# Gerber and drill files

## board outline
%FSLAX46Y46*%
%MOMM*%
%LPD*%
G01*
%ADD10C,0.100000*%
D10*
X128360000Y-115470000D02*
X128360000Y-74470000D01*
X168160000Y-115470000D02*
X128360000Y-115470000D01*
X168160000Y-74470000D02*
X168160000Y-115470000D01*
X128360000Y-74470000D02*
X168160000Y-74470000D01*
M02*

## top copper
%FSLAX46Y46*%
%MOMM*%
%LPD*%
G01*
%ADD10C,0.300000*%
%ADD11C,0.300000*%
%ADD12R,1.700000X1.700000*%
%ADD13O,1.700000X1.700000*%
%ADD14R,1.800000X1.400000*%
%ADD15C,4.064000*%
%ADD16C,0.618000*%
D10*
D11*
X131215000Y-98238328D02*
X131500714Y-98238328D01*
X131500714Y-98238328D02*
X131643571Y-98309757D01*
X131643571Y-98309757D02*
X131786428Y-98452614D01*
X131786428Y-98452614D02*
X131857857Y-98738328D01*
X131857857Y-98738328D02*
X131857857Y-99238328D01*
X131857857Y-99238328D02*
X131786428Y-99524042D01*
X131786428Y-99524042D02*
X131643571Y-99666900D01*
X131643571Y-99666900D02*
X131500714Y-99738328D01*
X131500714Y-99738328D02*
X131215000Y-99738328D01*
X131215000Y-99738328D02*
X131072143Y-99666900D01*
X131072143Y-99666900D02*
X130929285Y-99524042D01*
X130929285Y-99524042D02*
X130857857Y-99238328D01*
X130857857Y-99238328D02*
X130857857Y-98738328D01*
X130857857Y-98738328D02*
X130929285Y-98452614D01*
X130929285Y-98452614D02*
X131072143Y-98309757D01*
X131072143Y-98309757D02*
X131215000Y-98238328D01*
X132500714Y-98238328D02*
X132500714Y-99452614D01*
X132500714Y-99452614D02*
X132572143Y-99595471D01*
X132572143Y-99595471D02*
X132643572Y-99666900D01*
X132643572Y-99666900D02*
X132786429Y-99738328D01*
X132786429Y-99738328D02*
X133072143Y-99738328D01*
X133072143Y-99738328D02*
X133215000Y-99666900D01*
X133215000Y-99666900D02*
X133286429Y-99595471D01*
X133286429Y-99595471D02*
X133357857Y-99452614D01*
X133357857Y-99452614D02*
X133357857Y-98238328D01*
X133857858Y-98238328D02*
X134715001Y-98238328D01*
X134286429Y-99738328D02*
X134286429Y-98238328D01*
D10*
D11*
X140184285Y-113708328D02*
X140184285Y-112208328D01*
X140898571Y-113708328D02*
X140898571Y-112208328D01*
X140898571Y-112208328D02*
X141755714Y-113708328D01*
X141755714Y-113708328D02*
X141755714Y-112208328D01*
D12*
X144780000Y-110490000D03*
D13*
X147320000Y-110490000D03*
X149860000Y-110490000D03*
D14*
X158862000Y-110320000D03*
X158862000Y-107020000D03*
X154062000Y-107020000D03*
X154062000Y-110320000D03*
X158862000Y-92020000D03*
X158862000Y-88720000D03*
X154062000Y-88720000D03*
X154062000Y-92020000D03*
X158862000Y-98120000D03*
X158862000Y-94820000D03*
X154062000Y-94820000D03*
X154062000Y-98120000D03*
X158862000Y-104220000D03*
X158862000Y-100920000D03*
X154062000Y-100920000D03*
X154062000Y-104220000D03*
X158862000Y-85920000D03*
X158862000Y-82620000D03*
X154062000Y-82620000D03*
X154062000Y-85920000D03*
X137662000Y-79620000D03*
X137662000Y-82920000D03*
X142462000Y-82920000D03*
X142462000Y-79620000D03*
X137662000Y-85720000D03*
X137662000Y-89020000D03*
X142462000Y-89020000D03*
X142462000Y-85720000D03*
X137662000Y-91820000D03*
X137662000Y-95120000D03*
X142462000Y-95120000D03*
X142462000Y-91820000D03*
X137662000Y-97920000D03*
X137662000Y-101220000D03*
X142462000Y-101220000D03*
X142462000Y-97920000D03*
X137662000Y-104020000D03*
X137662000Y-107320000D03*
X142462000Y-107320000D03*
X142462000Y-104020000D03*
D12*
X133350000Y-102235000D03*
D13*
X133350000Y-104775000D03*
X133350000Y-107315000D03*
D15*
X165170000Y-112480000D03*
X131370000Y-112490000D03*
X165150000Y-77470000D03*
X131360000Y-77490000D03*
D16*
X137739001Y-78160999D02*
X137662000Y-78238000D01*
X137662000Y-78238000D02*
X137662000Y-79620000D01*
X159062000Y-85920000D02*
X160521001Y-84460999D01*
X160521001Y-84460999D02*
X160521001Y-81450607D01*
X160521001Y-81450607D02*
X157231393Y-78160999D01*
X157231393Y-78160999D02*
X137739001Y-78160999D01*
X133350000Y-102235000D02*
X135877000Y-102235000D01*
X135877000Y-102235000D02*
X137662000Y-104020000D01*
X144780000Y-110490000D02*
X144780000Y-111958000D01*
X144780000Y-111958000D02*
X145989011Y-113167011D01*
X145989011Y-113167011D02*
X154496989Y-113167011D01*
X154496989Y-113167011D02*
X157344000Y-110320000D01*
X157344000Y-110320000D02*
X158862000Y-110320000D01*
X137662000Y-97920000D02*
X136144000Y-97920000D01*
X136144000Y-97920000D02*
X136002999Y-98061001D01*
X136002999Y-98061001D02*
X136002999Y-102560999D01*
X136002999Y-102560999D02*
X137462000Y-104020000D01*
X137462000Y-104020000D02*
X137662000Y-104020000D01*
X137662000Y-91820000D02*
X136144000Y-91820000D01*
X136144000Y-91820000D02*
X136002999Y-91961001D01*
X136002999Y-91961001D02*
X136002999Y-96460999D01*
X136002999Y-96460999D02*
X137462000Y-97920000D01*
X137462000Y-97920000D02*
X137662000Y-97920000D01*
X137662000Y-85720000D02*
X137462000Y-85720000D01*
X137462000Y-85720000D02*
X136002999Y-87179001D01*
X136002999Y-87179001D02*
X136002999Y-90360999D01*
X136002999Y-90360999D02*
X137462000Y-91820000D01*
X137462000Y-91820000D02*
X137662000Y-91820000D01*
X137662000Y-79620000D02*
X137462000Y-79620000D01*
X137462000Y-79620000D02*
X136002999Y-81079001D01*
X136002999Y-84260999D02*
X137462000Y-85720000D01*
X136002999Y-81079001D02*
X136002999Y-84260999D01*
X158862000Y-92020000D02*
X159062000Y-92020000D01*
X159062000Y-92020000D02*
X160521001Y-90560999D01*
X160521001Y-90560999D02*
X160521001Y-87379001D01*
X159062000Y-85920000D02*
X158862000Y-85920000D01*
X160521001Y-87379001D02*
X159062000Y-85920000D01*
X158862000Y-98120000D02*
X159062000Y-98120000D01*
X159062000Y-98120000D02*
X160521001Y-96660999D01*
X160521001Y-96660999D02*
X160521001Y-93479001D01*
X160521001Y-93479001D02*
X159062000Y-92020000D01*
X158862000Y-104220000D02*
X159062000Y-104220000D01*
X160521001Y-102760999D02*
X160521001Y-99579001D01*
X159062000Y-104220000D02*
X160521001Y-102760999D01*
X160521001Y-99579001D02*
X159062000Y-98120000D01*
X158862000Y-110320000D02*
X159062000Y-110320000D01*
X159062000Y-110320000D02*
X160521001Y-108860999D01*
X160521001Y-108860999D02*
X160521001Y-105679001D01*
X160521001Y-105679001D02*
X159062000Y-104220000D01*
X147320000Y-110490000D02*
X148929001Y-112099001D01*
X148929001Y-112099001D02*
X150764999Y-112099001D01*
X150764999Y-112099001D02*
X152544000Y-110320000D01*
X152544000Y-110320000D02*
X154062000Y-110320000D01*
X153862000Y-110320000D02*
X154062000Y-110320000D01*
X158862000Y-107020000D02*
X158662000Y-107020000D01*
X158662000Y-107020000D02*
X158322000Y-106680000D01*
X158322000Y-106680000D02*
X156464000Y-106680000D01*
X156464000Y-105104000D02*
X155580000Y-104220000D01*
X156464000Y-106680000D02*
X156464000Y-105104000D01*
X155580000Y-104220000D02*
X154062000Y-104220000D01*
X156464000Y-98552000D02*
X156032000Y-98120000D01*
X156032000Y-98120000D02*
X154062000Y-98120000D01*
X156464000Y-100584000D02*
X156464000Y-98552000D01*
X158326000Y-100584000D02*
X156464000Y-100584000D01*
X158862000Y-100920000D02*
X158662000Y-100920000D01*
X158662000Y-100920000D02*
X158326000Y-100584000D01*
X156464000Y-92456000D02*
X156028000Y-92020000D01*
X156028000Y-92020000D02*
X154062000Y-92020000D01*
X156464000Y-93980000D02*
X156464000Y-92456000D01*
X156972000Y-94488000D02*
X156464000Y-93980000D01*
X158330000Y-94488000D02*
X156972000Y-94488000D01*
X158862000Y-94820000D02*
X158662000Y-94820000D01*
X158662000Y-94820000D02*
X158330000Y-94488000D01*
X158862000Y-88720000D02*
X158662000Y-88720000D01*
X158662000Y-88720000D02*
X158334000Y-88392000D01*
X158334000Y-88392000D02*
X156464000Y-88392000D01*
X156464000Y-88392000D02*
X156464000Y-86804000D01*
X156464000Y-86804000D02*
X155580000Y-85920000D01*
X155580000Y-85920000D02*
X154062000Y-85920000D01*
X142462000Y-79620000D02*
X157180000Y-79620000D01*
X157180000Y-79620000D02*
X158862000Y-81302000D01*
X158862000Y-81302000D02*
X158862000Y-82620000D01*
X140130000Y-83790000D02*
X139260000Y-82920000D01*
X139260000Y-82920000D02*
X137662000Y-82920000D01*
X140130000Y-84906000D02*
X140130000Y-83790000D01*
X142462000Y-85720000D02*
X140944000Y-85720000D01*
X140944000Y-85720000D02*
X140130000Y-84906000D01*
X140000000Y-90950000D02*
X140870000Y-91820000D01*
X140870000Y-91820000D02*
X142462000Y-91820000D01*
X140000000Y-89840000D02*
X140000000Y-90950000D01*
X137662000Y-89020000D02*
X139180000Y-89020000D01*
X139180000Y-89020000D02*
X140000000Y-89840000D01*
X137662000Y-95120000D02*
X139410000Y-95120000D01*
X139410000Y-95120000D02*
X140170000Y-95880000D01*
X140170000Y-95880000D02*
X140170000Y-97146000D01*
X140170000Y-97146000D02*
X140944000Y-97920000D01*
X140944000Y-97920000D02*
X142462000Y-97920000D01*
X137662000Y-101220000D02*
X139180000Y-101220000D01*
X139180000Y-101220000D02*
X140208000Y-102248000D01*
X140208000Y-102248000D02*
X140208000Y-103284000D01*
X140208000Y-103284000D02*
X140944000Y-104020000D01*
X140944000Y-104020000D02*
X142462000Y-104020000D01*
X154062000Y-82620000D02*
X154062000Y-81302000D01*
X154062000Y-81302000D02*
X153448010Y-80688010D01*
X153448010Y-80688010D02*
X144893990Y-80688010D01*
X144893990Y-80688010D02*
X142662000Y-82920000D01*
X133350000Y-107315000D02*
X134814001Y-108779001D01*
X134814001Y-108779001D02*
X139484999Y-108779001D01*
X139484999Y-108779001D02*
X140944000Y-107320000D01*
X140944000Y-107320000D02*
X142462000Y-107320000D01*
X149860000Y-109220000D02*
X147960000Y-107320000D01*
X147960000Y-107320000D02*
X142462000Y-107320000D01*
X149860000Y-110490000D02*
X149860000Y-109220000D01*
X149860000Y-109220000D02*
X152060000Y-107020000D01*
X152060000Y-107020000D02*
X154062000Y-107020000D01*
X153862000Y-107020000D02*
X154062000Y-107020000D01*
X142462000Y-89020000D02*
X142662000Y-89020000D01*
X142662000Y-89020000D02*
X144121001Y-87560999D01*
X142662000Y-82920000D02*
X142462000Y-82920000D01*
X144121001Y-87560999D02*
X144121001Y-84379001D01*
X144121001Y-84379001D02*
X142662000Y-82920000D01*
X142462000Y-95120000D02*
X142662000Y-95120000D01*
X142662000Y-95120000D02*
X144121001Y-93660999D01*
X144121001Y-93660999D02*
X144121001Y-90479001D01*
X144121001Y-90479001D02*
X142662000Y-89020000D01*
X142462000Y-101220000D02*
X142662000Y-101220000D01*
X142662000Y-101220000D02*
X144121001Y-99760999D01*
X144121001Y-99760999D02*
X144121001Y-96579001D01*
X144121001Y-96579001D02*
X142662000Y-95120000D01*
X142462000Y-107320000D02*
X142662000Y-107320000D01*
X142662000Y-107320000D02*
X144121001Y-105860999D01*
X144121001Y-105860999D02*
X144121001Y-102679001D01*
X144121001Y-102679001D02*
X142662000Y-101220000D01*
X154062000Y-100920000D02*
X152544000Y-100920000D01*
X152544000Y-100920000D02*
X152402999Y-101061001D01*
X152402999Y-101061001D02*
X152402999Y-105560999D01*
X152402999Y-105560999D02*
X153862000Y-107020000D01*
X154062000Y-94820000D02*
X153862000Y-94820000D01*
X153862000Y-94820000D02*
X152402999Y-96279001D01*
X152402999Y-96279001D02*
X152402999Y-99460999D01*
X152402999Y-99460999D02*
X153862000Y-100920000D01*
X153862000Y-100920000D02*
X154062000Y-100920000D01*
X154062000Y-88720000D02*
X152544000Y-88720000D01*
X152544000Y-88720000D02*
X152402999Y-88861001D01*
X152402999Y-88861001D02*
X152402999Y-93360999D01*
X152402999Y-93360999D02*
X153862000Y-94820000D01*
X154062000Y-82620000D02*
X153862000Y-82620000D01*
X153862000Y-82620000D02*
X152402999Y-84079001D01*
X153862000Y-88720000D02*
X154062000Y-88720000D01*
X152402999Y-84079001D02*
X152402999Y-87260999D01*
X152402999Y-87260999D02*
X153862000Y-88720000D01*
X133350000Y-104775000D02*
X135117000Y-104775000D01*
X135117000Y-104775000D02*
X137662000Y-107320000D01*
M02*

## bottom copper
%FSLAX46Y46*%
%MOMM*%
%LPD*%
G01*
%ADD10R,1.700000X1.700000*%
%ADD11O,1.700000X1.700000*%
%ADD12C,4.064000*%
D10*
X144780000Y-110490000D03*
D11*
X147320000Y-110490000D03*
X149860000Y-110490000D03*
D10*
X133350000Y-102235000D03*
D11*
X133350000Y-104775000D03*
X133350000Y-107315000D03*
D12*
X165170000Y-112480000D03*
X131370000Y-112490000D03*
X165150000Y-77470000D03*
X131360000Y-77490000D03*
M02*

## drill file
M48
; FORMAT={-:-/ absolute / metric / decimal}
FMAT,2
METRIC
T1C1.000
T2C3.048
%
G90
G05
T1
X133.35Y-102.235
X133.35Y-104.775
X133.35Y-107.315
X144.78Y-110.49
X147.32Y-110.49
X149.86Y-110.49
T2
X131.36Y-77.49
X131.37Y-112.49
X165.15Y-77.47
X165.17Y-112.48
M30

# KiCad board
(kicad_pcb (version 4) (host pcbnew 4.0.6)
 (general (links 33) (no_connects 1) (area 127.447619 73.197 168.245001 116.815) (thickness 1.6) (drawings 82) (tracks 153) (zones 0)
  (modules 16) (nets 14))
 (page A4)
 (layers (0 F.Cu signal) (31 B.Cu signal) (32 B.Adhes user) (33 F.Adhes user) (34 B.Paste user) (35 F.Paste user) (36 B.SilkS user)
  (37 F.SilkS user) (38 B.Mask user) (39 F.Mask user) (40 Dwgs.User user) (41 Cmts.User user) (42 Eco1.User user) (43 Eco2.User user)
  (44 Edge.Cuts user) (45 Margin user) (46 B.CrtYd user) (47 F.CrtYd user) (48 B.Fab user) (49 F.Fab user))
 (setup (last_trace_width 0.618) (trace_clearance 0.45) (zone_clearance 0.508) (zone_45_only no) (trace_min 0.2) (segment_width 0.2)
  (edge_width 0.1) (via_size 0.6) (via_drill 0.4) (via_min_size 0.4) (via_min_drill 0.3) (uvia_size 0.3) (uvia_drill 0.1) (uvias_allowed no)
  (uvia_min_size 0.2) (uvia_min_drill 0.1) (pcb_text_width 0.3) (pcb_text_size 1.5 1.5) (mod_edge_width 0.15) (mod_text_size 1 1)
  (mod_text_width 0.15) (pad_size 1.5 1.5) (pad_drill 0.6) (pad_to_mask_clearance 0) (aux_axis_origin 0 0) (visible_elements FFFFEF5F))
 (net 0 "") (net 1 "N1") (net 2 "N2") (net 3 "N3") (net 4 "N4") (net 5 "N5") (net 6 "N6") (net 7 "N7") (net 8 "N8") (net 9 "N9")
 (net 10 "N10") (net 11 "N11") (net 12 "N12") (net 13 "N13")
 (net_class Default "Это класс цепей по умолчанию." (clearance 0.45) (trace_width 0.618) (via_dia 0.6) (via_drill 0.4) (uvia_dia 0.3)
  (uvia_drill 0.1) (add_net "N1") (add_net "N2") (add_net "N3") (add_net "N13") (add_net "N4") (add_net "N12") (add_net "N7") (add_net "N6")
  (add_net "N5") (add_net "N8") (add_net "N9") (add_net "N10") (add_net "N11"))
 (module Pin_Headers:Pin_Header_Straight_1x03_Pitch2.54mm (layer F.Cu) (at 144.78 110.49 90)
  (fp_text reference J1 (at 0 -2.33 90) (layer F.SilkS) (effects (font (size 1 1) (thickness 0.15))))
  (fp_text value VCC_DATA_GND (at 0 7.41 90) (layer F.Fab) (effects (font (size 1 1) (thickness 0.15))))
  (pad 1 thru_hole rect (at 0 0 90) (size 1.7 1.7) (drill 1) (layers *.Cu *.Mask) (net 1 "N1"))
  (pad 2 thru_hole oval (at 0 2.54 90) (size 1.7 1.7) (drill 1) (layers *.Cu *.Mask) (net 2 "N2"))
  (pad 3 thru_hole oval (at 0 5.08 90) (size 1.7 1.7) (drill 1) (layers *.Cu *.Mask) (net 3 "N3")))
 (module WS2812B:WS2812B (layer F.Cu) (at 156.462 108.67 270)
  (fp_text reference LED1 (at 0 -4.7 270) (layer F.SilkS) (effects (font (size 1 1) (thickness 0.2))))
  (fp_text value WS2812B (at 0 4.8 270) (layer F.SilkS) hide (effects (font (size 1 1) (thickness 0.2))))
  (pad 1 smd rect (at 1.65 -2.4 270) (size 1.4 1.8) (layers F.Cu F.Paste F.Mask) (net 1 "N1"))
  (pad 2 smd rect (at -1.65 -2.4 270) (size 1.4 1.8) (layers F.Cu F.Paste F.Mask) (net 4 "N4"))
  (pad 3 smd rect (at -1.65 2.4 270) (size 1.4 1.8) (layers F.Cu F.Paste F.Mask) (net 3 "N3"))
  (pad 4 smd rect (at 1.65 2.4 270) (size 1.4 1.8) (layers F.Cu F.Paste F.Mask) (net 2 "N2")))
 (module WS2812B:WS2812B (layer F.Cu) (at 156.462 90.37 270)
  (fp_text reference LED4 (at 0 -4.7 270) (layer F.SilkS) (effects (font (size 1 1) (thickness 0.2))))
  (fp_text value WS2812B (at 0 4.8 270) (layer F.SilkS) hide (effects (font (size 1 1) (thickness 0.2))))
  (pad 1 smd rect (at 1.65 -2.4 270) (size 1.4 1.8) (layers F.Cu F.Paste F.Mask) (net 1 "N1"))
  (pad 2 smd rect (at -1.65 -2.4 270) (size 1.4 1.8) (layers F.Cu F.Paste F.Mask) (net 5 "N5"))
  (pad 3 smd rect (at -1.65 2.4 270) (size 1.4 1.8) (layers F.Cu F.Paste F.Mask) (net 3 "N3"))
  (pad 4 smd rect (at 1.65 2.4 270) (size 1.4 1.8) (layers F.Cu F.Paste F.Mask) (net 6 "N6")))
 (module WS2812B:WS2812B (layer F.Cu) (at 156.462 96.47 270)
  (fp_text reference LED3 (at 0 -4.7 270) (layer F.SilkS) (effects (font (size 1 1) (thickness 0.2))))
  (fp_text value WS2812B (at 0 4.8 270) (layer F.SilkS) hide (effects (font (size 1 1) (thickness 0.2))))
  (pad 1 smd rect (at 1.65 -2.4 270) (size 1.4 1.8) (layers F.Cu F.Paste F.Mask) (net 1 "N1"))
  (pad 2 smd rect (at -1.65 -2.4 270) (size 1.4 1.8) (layers F.Cu F.Paste F.Mask) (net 6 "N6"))
  (pad 3 smd rect (at -1.65 2.4 270) (size 1.4 1.8) (layers F.Cu F.Paste F.Mask) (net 3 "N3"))
  (pad 4 smd rect (at 1.65 2.4 270) (size 1.4 1.8) (layers F.Cu F.Paste F.Mask) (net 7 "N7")))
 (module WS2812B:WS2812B (layer F.Cu) (at 156.462 102.57 270)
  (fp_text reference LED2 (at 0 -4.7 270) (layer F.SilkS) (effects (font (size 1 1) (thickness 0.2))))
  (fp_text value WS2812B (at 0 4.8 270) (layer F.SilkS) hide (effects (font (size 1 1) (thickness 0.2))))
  (pad 1 smd rect (at 1.65 -2.4 270) (size 1.4 1.8) (layers F.Cu F.Paste F.Mask) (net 1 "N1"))
  (pad 2 smd rect (at -1.65 -2.4 270) (size 1.4 1.8) (layers F.Cu F.Paste F.Mask) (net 7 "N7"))
  (pad 3 smd rect (at -1.65 2.4 270) (size 1.4 1.8) (layers F.Cu F.Paste F.Mask) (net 3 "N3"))
  (pad 4 smd rect (at 1.65 2.4 270) (size 1.4 1.8) (layers F.Cu F.Paste F.Mask) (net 4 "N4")))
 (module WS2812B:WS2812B (layer F.Cu) (at 156.462 84.27 270)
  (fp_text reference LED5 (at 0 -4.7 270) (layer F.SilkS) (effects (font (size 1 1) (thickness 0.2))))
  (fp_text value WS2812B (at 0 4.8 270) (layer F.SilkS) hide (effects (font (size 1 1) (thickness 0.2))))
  (pad 1 smd rect (at 1.65 -2.4 270) (size 1.4 1.8) (layers F.Cu F.Paste F.Mask) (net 1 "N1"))
  (pad 2 smd rect (at -1.65 -2.4 270) (size 1.4 1.8) (layers F.Cu F.Paste F.Mask) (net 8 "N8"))
  (pad 3 smd rect (at -1.65 2.4 270) (size 1.4 1.8) (layers F.Cu F.Paste F.Mask) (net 3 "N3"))
  (pad 4 smd rect (at 1.65 2.4 270) (size 1.4 1.8) (layers F.Cu F.Paste F.Mask) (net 5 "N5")))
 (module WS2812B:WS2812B (layer F.Cu) (at 140.062 81.27 90)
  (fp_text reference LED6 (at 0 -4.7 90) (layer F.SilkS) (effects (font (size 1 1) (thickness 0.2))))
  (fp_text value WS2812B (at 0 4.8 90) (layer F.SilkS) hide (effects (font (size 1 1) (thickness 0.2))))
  (pad 1 smd rect (at 1.65 -2.4 90) (size 1.4 1.8) (layers F.Cu F.Paste F.Mask) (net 1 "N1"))
  (pad 2 smd rect (at -1.65 -2.4 90) (size 1.4 1.8) (layers F.Cu F.Paste F.Mask) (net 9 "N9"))
  (pad 3 smd rect (at -1.65 2.4 90) (size 1.4 1.8) (layers F.Cu F.Paste F.Mask) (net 3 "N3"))
  (pad 4 smd rect (at 1.65 2.4 90) (size 1.4 1.8) (layers F.Cu F.Paste F.Mask) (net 8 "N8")))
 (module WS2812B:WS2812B (layer F.Cu) (at 140.062 87.37 90)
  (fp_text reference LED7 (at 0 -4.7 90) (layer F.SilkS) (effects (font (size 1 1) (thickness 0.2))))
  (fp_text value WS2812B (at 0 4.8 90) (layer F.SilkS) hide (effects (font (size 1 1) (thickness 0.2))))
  (pad 1 smd rect (at 1.65 -2.4 90) (size 1.4 1.8) (layers F.Cu F.Paste F.Mask) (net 1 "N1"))
  (pad 2 smd rect (at -1.65 -2.4 90) (size 1.4 1.8) (layers F.Cu F.Paste F.Mask) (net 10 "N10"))
  (pad 3 smd rect (at -1.65 2.4 90) (size 1.4 1.8) (layers F.Cu F.Paste F.Mask) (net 3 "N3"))
  (pad 4 smd rect (at 1.65 2.4 90) (size 1.4 1.8) (layers F.Cu F.Paste F.Mask) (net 9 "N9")))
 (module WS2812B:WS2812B (layer F.Cu) (at 140.062 93.47 90)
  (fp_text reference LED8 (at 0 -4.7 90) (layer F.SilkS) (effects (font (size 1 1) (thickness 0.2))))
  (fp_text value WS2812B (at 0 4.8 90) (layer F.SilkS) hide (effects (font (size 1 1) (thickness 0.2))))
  (pad 1 smd rect (at 1.65 -2.4 90) (size 1.4 1.8) (layers F.Cu F.Paste F.Mask) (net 1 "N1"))
  (pad 2 smd rect (at -1.65 -2.4 90) (size 1.4 1.8) (layers F.Cu F.Paste F.Mask) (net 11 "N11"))
  (pad 3 smd rect (at -1.65 2.4 90) (size 1.4 1.8) (layers F.Cu F.Paste F.Mask) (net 3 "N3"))
  (pad 4 smd rect (at 1.65 2.4 90) (size 1.4 1.8) (layers F.Cu F.Paste F.Mask) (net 10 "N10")))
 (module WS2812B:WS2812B (layer F.Cu) (at 140.062 99.57 90)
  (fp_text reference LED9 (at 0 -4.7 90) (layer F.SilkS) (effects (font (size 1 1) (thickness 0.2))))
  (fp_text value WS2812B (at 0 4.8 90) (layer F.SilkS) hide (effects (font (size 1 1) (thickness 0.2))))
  (pad 1 smd rect (at 1.65 -2.4 90) (size 1.4 1.8) (layers F.Cu F.Paste F.Mask) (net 1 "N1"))
  (pad 2 smd rect (at -1.65 -2.4 90) (size 1.4 1.8) (layers F.Cu F.Paste F.Mask) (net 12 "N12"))
  (pad 3 smd rect (at -1.65 2.4 90) (size 1.4 1.8) (layers F.Cu F.Paste F.Mask) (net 3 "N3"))
  (pad 4 smd rect (at 1.65 2.4 90) (size 1.4 1.8) (layers F.Cu F.Paste F.Mask) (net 11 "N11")))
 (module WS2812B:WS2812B (layer F.Cu) (at 140.062 105.67 90)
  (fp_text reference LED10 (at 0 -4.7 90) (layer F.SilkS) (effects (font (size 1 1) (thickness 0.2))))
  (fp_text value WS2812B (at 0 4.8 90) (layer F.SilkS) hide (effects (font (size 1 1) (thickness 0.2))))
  (pad 1 smd rect (at 1.65 -2.4 90) (size 1.4 1.8) (layers F.Cu F.Paste F.Mask) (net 1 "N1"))
  (pad 2 smd rect (at -1.65 -2.4 90) (size 1.4 1.8) (layers F.Cu F.Paste F.Mask) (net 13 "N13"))
  (pad 3 smd rect (at -1.65 2.4 90) (size 1.4 1.8) (layers F.Cu F.Paste F.Mask) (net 3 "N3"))
  (pad 4 smd rect (at 1.65 2.4 90) (size 1.4 1.8) (layers F.Cu F.Paste F.Mask) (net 12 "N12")))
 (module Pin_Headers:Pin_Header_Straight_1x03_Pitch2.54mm (layer F.Cu) (at 133.35 102.235)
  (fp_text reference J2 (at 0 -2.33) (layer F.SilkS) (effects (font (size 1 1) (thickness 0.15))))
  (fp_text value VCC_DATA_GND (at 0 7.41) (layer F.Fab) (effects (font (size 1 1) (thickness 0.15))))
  (pad 1 thru_hole rect (at 0 0) (size 1.7 1.7) (drill 1) (layers *.Cu *.Mask) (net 1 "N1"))
  (pad 2 thru_hole oval (at 0 2.54) (size 1.7 1.7) (drill 1) (layers *.Cu *.Mask) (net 13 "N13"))
  (pad 3 thru_hole oval (at 0 5.08) (size 1.7 1.7) (drill 1) (layers *.Cu *.Mask) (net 3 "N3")))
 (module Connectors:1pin (layer F.Cu) (at 165.17 112.48)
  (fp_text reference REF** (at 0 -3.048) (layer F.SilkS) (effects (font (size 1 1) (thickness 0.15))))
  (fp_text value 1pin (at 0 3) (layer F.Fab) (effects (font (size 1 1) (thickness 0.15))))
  (pad 1 thru_hole circle (at 0 0) (size 4.064 4.064) (drill 3.048) (layers *.Cu *.Mask)))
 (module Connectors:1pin (layer F.Cu) (at 131.37 112.49)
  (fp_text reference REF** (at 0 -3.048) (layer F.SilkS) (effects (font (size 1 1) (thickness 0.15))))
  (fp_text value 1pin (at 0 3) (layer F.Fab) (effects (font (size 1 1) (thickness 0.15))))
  (pad 1 thru_hole circle (at 0 0) (size 4.064 4.064) (drill 3.048) (layers *.Cu *.Mask)))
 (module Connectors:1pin (layer F.Cu) (at 165.15 77.47)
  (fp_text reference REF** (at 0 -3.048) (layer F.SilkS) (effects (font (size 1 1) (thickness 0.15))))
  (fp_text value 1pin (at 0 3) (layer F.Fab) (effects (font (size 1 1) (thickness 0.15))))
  (pad 1 thru_hole circle (at 0 0) (size 4.064 4.064) (drill 3.048) (layers *.Cu *.Mask)))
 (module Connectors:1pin (layer F.Cu) (at 131.36 77.49)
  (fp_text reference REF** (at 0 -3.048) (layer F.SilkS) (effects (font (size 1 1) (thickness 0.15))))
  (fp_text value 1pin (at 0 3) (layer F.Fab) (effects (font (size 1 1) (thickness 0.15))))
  (pad 1 thru_hole circle (at 0 0) (size 4.064 4.064) (drill 3.048) (layers *.Cu *.Mask)))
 (gr_line (start 128.36 115.47) (end 128.36 74.47) (layer Edge.Cuts) (width 0.1))
 (gr_line (start 168.16 115.47) (end 128.36 115.47) (layer Edge.Cuts) (width 0.1))
 (gr_line (start 168.16 74.47) (end 168.16 115.47) (layer Edge.Cuts) (width 0.1))
 (gr_line (start 128.36 74.47) (end 168.16 74.47) (layer Edge.Cuts) (width 0.1))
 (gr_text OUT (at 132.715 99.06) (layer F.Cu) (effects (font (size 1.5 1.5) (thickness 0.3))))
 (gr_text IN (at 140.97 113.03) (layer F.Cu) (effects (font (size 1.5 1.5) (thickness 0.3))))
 (segment (start 137.739001 78.160999) (end 137.662 78.238) (width 0.618) (layer F.Cu) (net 1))
 (segment (start 137.662 78.238) (end 137.662 79.62) (width 0.618) (layer F.Cu) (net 1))
 (segment (start 159.062 85.92) (end 160.521001 84.460999) (width 0.618) (layer F.Cu) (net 1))
 (segment (start 160.521001 84.460999) (end 160.521001 81.450607) (width 0.618) (layer F.Cu) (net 1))
 (segment (start 160.521001 81.450607) (end 157.231393 78.160999) (width 0.618) (layer F.Cu) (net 1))
 (segment (start 157.231393 78.160999) (end 137.739001 78.160999) (width 0.618) (layer F.Cu) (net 1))
 (segment (start 133.35 102.235) (end 135.877 102.235) (width 0.618) (layer F.Cu) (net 1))
 (segment (start 135.877 102.235) (end 137.662 104.02) (width 0.618) (layer F.Cu) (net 1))
 (segment (start 144.78 110.49) (end 144.78 111.958) (width 0.618) (layer F.Cu) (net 1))
 (segment (start 144.78 111.958) (end 145.989011 113.167011) (width 0.618) (layer F.Cu) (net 1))
 (segment (start 145.989011 113.167011) (end 154.496989 113.167011) (width 0.618) (layer F.Cu) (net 1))
 (segment (start 154.496989 113.167011) (end 157.344 110.32) (width 0.618) (layer F.Cu) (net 1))
 (segment (start 157.344 110.32) (end 158.862 110.32) (width 0.618) (layer F.Cu) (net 1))
 (segment (start 137.662 97.92) (end 136.144 97.92) (width 0.618) (layer F.Cu) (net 1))
 (segment (start 136.144 97.92) (end 136.002999 98.061001) (width 0.618) (layer F.Cu) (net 1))
 (segment (start 136.002999 98.061001) (end 136.002999 102.560999) (width 0.618) (layer F.Cu) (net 1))
 (segment (start 136.002999 102.560999) (end 137.462 104.02) (width 0.618) (layer F.Cu) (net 1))
 (segment (start 137.462 104.02) (end 137.662 104.02) (width 0.618) (layer F.Cu) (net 1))
 (segment (start 137.662 91.82) (end 136.144 91.82) (width 0.618) (layer F.Cu) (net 1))
 (segment (start 136.144 91.82) (end 136.002999 91.961001) (width 0.618) (layer F.Cu) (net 1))
 (segment (start 136.002999 91.961001) (end 136.002999 96.460999) (width 0.618) (layer F.Cu) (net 1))
 (segment (start 136.002999 96.460999) (end 137.462 97.92) (width 0.618) (layer F.Cu) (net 1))
 (segment (start 137.462 97.92) (end 137.662 97.92) (width 0.618) (layer F.Cu) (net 1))
 (segment (start 137.662 85.72) (end 137.462 85.72) (width 0.618) (layer F.Cu) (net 1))
 (segment (start 137.462 85.72) (end 136.002999 87.179001) (width 0.618) (layer F.Cu) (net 1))
 (segment (start 136.002999 87.179001) (end 136.002999 90.360999) (width 0.618) (layer F.Cu) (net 1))
 (segment (start 136.002999 90.360999) (end 137.462 91.82) (width 0.618) (layer F.Cu) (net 1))
 (segment (start 137.462 91.82) (end 137.662 91.82) (width 0.618) (layer F.Cu) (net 1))
 (segment (start 137.662 79.62) (end 137.462 79.62) (width 0.618) (layer F.Cu) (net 1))
 (segment (start 137.462 79.62) (end 136.002999 81.079001) (width 0.618) (layer F.Cu) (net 1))
 (segment (start 136.002999 84.260999) (end 137.462 85.72) (width 0.618) (layer F.Cu) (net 1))
 (segment (start 136.002999 81.079001) (end 136.002999 84.260999) (width 0.618) (layer F.Cu) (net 1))
 (segment (start 158.862 92.02) (end 159.062 92.02) (width 0.618) (layer F.Cu) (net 1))
 (segment (start 159.062 92.02) (end 160.521001 90.560999) (width 0.618) (layer F.Cu) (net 1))
 (segment (start 160.521001 90.560999) (end 160.521001 87.379001) (width 0.618) (layer F.Cu) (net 1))
 (segment (start 159.062 85.92) (end 158.862 85.92) (width 0.618) (layer F.Cu) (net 1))
 (segment (start 160.521001 87.379001) (end 159.062 85.92) (width 0.618) (layer F.Cu) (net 1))
 (segment (start 158.862 98.12) (end 159.062 98.12) (width 0.618) (layer F.Cu) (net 1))
 (segment (start 159.062 98.12) (end 160.521001 96.660999) (width 0.618) (layer F.Cu) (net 1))
 (segment (start 160.521001 96.660999) (end 160.521001 93.479001) (width 0.618) (layer F.Cu) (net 1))
 (segment (start 160.521001 93.479001) (end 159.062 92.02) (width 0.618) (layer F.Cu) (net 1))
 (segment (start 158.862 104.22) (end 159.062 104.22) (width 0.618) (layer F.Cu) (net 1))
 (segment (start 160.521001 102.760999) (end 160.521001 99.579001) (width 0.618) (layer F.Cu) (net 1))
 (segment (start 159.062 104.22) (end 160.521001 102.760999) (width 0.618) (layer F.Cu) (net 1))
 (segment (start 160.521001 99.579001) (end 159.062 98.12) (width 0.618) (layer F.Cu) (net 1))
 (segment (start 158.862 110.32) (end 159.062 110.32) (width 0.618) (layer F.Cu) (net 1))
 (segment (start 159.062 110.32) (end 160.521001 108.860999) (width 0.618) (layer F.Cu) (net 1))
 (segment (start 160.521001 108.860999) (end 160.521001 105.679001) (width 0.618) (layer F.Cu) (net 1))
 (segment (start 160.521001 105.679001) (end 159.062 104.22) (width 0.618) (layer F.Cu) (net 1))
 (segment (start 147.32 110.49) (end 148.929001 112.099001) (width 0.618) (layer F.Cu) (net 2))
 (segment (start 148.929001 112.099001) (end 150.764999 112.099001) (width 0.618) (layer F.Cu) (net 2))
 (segment (start 150.764999 112.099001) (end 152.544 110.32) (width 0.618) (layer F.Cu) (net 2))
 (segment (start 152.544 110.32) (end 154.062 110.32) (width 0.618) (layer F.Cu) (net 2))
 (segment (start 153.862 110.32) (end 154.062 110.32) (width 0.618) (layer F.Cu) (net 2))
 (segment (start 158.862 107.02) (end 158.662 107.02) (width 0.618) (layer F.Cu) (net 4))
 (segment (start 158.662 107.02) (end 158.322 106.68) (width 0.618) (layer F.Cu) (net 4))
 (segment (start 158.322 106.68) (end 156.464 106.68) (width 0.618) (layer F.Cu) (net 4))
 (segment (start 156.464 105.104) (end 155.58 104.22) (width 0.618) (layer F.Cu) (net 4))
 (segment (start 156.464 106.68) (end 156.464 105.104) (width 0.618) (layer F.Cu) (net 4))
 (segment (start 155.58 104.22) (end 154.062 104.22) (width 0.618) (layer F.Cu) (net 4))
 (segment (start 156.464 98.552) (end 156.032 98.12) (width 0.618) (layer F.Cu) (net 7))
 (segment (start 156.032 98.12) (end 154.062 98.12) (width 0.618) (layer F.Cu) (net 7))
 (segment (start 156.464 100.584) (end 156.464 98.552) (width 0.618) (layer F.Cu) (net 7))
 (segment (start 158.326 100.584) (end 156.464 100.584) (width 0.618) (layer F.Cu) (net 7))
 (segment (start 158.862 100.92) (end 158.662 100.92) (width 0.618) (layer F.Cu) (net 7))
 (segment (start 158.662 100.92) (end 158.326 100.584) (width 0.618) (layer F.Cu) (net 7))
 (segment (start 156.464 92.456) (end 156.028 92.02) (width 0.618) (layer F.Cu) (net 6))
 (segment (start 156.028 92.02) (end 154.062 92.02) (width 0.618) (layer F.Cu) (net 6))
 (segment (start 156.464 93.98) (end 156.464 92.456) (width 0.618) (layer F.Cu) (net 6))
 (segment (start 156.972 94.488) (end 156.464 93.98) (width 0.618) (layer F.Cu) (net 6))
 (segment (start 158.33 94.488) (end 156.972 94.488) (width 0.618) (layer F.Cu) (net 6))
 (segment (start 158.862 94.82) (end 158.662 94.82) (width 0.618) (layer F.Cu) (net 6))
 (segment (start 158.662 94.82) (end 158.33 94.488) (width 0.618) (layer F.Cu) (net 6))
 (segment (start 158.862 88.72) (end 158.662 88.72) (width 0.618) (layer F.Cu) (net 5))
 (segment (start 158.662 88.72) (end 158.334 88.392) (width 0.618) (layer F.Cu) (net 5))
 (segment (start 158.334 88.392) (end 156.464 88.392) (width 0.618) (layer F.Cu) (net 5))
 (segment (start 156.464 88.392) (end 156.464 86.804) (width 0.618) (layer F.Cu) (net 5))
 (segment (start 156.464 86.804) (end 155.58 85.92) (width 0.618) (layer F.Cu) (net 5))
 (segment (start 155.58 85.92) (end 154.062 85.92) (width 0.618) (layer F.Cu) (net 5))
 (segment (start 142.462 79.62) (end 157.18 79.62) (width 0.618) (layer F.Cu) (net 8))
 (segment (start 157.18 79.62) (end 158.862 81.302) (width 0.618) (layer F.Cu) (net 8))
 (segment (start 158.862 81.302) (end 158.862 82.62) (width 0.618) (layer F.Cu) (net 8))
 (segment (start 140.13 83.79) (end 139.26 82.92) (width 0.618) (layer F.Cu) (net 9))
 (segment (start 139.26 82.92) (end 137.662 82.92) (width 0.618) (layer F.Cu) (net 9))
 (segment (start 140.13 84.906) (end 140.13 83.79) (width 0.618) (layer F.Cu) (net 9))
 (segment (start 142.462 85.72) (end 140.944 85.72) (width 0.618) (layer F.Cu) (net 9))
 (segment (start 140.944 85.72) (end 140.13 84.906) (width 0.618) (layer F.Cu) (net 9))
 (segment (start 140 90.95) (end 140.87 91.82) (width 0.618) (layer F.Cu) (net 10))
 (segment (start 140.87 91.82) (end 142.462 91.82) (width 0.618) (layer F.Cu) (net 10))
 (segment (start 140 89.84) (end 140 90.95) (width 0.618) (layer F.Cu) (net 10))
 (segment (start 137.662 89.02) (end 139.18 89.02) (width 0.618) (layer F.Cu) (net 10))
 (segment (start 139.18 89.02) (end 140 89.84) (width 0.618) (layer F.Cu) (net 10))
 (segment (start 137.662 95.12) (end 139.41 95.12) (width 0.618) (layer F.Cu) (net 11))
 (segment (start 139.41 95.12) (end 140.17 95.88) (width 0.618) (layer F.Cu) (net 11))
 (segment (start 140.17 95.88) (end 140.17 97.146) (width 0.618) (layer F.Cu) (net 11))
 (segment (start 140.17 97.146) (end 140.944 97.92) (width 0.618) (layer F.Cu) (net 11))
 (segment (start 140.944 97.92) (end 142.462 97.92) (width 0.618) (layer F.Cu) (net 11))
 (segment (start 137.662 101.22) (end 139.18 101.22) (width 0.618) (layer F.Cu) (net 12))
 (segment (start 139.18 101.22) (end 140.208 102.248) (width 0.618) (layer F.Cu) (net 12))
 (segment (start 140.208 102.248) (end 140.208 103.284) (width 0.618) (layer F.Cu) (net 12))
 (segment (start 140.208 103.284) (end 140.944 104.02) (width 0.618) (layer F.Cu) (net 12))
 (segment (start 140.944 104.02) (end 142.462 104.02) (width 0.618) (layer F.Cu) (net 12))
 (segment (start 154.062 82.62) (end 154.062 81.302) (width 0.618) (layer F.Cu) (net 3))
 (segment (start 154.062 81.302) (end 153.44801 80.68801) (width 0.618) (layer F.Cu) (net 3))
 (segment (start 153.44801 80.68801) (end 144.89399 80.68801) (width 0.618) (layer F.Cu) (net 3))
 (segment (start 144.89399 80.68801) (end 142.662 82.92) (width 0.618) (layer F.Cu) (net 3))
 (segment (start 133.35 107.315) (end 134.814001 108.779001) (width 0.618) (layer F.Cu) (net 3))
 (segment (start 134.814001 108.779001) (end 139.484999 108.779001) (width 0.618) (layer F.Cu) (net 3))
 (segment (start 139.484999 108.779001) (end 140.944 107.32) (width 0.618) (layer F.Cu) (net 3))
 (segment (start 140.944 107.32) (end 142.462 107.32) (width 0.618) (layer F.Cu) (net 3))
 (segment (start 149.86 109.22) (end 147.96 107.32) (width 0.618) (layer F.Cu) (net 3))
 (segment (start 147.96 107.32) (end 142.462 107.32) (width 0.618) (layer F.Cu) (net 3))
 (segment (start 149.86 110.49) (end 149.86 109.22) (width 0.618) (layer F.Cu) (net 3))
 (segment (start 149.86 109.22) (end 152.06 107.02) (width 0.618) (layer F.Cu) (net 3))
 (segment (start 152.06 107.02) (end 154.062 107.02) (width 0.618) (layer F.Cu) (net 3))
 (segment (start 153.862 107.02) (end 154.062 107.02) (width 0.618) (layer F.Cu) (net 3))
 (segment (start 142.462 89.02) (end 142.662 89.02) (width 0.618) (layer F.Cu) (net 3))
 (segment (start 142.662 89.02) (end 144.121001 87.560999) (width 0.618) (layer F.Cu) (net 3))
 (segment (start 142.662 82.92) (end 142.462 82.92) (width 0.618) (layer F.Cu) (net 3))
 (segment (start 144.121001 87.560999) (end 144.121001 84.379001) (width 0.618) (layer F.Cu) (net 3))
 (segment (start 144.121001 84.379001) (end 142.662 82.92) (width 0.618) (layer F.Cu) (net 3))
 (segment (start 142.462 95.12) (end 142.662 95.12) (width 0.618) (layer F.Cu) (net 3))
 (segment (start 142.662 95.12) (end 144.121001 93.660999) (width 0.618) (layer F.Cu) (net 3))
 (segment (start 144.121001 93.660999) (end 144.121001 90.479001) (width 0.618) (layer F.Cu) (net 3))
 (segment (start 144.121001 90.479001) (end 142.662 89.02) (width 0.618) (layer F.Cu) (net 3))
 (segment (start 142.462 101.22) (end 142.662 101.22) (width 0.618) (layer F.Cu) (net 3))
 (segment (start 142.662 101.22) (end 144.121001 99.760999) (width 0.618) (layer F.Cu) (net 3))
 (segment (start 144.121001 99.760999) (end 144.121001 96.579001) (width 0.618) (layer F.Cu) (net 3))
 (segment (start 144.121001 96.579001) (end 142.662 95.12) (width 0.618) (layer F.Cu) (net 3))
 (segment (start 142.462 107.32) (end 142.662 107.32) (width 0.618) (layer F.Cu) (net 3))
 (segment (start 142.662 107.32) (end 144.121001 105.860999) (width 0.618) (layer F.Cu) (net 3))
 (segment (start 144.121001 105.860999) (end 144.121001 102.679001) (width 0.618) (layer F.Cu) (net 3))
 (segment (start 144.121001 102.679001) (end 142.662 101.22) (width 0.618) (layer F.Cu) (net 3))
 (segment (start 154.062 100.92) (end 152.544 100.92) (width 0.618) (layer F.Cu) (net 3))
 (segment (start 152.544 100.92) (end 152.402999 101.061001) (width 0.618) (layer F.Cu) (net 3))
 (segment (start 152.402999 101.061001) (end 152.402999 105.560999) (width 0.618) (layer F.Cu) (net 3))
 (segment (start 152.402999 105.560999) (end 153.862 107.02) (width 0.618) (layer F.Cu) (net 3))
 (segment (start 154.062 94.82) (end 153.862 94.82) (width 0.618) (layer F.Cu) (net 3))
 (segment (start 153.862 94.82) (end 152.402999 96.279001) (width 0.618) (layer F.Cu) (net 3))
 (segment (start 152.402999 96.279001) (end 152.402999 99.460999) (width 0.618) (layer F.Cu) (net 3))
 (segment (start 152.402999 99.460999) (end 153.862 100.92) (width 0.618) (layer F.Cu) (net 3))
 (segment (start 153.862 100.92) (end 154.062 100.92) (width 0.618) (layer F.Cu) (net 3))
 (segment (start 154.062 88.72) (end 152.544 88.72) (width 0.618) (layer F.Cu) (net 3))
 (segment (start 152.544 88.72) (end 152.402999 88.861001) (width 0.618) (layer F.Cu) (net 3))
 (segment (start 152.402999 88.861001) (end 152.402999 93.360999) (width 0.618) (layer F.Cu) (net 3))
 (segment (start 152.402999 93.360999) (end 153.862 94.82) (width 0.618) (layer F.Cu) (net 3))
 (segment (start 154.062 82.62) (end 153.862 82.62) (width 0.618) (layer F.Cu) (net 3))
 (segment (start 153.862 82.62) (end 152.402999 84.079001) (width 0.618) (layer F.Cu) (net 3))
 (segment (start 153.862 88.72) (end 154.062 88.72) (width 0.618) (layer F.Cu) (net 3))
 (segment (start 152.402999 84.079001) (end 152.402999 87.260999) (width 0.618) (layer F.Cu) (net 3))
 (segment (start 152.402999 87.260999) (end 153.862 88.72) (width 0.618) (layer F.Cu) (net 3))
 (segment (start 133.35 104.775) (end 135.117 104.775) (width 0.618) (layer F.Cu) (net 13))
 (segment (start 135.117 104.775) (end 137.662 107.32) (width 0.618) (layer F.Cu) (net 13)))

